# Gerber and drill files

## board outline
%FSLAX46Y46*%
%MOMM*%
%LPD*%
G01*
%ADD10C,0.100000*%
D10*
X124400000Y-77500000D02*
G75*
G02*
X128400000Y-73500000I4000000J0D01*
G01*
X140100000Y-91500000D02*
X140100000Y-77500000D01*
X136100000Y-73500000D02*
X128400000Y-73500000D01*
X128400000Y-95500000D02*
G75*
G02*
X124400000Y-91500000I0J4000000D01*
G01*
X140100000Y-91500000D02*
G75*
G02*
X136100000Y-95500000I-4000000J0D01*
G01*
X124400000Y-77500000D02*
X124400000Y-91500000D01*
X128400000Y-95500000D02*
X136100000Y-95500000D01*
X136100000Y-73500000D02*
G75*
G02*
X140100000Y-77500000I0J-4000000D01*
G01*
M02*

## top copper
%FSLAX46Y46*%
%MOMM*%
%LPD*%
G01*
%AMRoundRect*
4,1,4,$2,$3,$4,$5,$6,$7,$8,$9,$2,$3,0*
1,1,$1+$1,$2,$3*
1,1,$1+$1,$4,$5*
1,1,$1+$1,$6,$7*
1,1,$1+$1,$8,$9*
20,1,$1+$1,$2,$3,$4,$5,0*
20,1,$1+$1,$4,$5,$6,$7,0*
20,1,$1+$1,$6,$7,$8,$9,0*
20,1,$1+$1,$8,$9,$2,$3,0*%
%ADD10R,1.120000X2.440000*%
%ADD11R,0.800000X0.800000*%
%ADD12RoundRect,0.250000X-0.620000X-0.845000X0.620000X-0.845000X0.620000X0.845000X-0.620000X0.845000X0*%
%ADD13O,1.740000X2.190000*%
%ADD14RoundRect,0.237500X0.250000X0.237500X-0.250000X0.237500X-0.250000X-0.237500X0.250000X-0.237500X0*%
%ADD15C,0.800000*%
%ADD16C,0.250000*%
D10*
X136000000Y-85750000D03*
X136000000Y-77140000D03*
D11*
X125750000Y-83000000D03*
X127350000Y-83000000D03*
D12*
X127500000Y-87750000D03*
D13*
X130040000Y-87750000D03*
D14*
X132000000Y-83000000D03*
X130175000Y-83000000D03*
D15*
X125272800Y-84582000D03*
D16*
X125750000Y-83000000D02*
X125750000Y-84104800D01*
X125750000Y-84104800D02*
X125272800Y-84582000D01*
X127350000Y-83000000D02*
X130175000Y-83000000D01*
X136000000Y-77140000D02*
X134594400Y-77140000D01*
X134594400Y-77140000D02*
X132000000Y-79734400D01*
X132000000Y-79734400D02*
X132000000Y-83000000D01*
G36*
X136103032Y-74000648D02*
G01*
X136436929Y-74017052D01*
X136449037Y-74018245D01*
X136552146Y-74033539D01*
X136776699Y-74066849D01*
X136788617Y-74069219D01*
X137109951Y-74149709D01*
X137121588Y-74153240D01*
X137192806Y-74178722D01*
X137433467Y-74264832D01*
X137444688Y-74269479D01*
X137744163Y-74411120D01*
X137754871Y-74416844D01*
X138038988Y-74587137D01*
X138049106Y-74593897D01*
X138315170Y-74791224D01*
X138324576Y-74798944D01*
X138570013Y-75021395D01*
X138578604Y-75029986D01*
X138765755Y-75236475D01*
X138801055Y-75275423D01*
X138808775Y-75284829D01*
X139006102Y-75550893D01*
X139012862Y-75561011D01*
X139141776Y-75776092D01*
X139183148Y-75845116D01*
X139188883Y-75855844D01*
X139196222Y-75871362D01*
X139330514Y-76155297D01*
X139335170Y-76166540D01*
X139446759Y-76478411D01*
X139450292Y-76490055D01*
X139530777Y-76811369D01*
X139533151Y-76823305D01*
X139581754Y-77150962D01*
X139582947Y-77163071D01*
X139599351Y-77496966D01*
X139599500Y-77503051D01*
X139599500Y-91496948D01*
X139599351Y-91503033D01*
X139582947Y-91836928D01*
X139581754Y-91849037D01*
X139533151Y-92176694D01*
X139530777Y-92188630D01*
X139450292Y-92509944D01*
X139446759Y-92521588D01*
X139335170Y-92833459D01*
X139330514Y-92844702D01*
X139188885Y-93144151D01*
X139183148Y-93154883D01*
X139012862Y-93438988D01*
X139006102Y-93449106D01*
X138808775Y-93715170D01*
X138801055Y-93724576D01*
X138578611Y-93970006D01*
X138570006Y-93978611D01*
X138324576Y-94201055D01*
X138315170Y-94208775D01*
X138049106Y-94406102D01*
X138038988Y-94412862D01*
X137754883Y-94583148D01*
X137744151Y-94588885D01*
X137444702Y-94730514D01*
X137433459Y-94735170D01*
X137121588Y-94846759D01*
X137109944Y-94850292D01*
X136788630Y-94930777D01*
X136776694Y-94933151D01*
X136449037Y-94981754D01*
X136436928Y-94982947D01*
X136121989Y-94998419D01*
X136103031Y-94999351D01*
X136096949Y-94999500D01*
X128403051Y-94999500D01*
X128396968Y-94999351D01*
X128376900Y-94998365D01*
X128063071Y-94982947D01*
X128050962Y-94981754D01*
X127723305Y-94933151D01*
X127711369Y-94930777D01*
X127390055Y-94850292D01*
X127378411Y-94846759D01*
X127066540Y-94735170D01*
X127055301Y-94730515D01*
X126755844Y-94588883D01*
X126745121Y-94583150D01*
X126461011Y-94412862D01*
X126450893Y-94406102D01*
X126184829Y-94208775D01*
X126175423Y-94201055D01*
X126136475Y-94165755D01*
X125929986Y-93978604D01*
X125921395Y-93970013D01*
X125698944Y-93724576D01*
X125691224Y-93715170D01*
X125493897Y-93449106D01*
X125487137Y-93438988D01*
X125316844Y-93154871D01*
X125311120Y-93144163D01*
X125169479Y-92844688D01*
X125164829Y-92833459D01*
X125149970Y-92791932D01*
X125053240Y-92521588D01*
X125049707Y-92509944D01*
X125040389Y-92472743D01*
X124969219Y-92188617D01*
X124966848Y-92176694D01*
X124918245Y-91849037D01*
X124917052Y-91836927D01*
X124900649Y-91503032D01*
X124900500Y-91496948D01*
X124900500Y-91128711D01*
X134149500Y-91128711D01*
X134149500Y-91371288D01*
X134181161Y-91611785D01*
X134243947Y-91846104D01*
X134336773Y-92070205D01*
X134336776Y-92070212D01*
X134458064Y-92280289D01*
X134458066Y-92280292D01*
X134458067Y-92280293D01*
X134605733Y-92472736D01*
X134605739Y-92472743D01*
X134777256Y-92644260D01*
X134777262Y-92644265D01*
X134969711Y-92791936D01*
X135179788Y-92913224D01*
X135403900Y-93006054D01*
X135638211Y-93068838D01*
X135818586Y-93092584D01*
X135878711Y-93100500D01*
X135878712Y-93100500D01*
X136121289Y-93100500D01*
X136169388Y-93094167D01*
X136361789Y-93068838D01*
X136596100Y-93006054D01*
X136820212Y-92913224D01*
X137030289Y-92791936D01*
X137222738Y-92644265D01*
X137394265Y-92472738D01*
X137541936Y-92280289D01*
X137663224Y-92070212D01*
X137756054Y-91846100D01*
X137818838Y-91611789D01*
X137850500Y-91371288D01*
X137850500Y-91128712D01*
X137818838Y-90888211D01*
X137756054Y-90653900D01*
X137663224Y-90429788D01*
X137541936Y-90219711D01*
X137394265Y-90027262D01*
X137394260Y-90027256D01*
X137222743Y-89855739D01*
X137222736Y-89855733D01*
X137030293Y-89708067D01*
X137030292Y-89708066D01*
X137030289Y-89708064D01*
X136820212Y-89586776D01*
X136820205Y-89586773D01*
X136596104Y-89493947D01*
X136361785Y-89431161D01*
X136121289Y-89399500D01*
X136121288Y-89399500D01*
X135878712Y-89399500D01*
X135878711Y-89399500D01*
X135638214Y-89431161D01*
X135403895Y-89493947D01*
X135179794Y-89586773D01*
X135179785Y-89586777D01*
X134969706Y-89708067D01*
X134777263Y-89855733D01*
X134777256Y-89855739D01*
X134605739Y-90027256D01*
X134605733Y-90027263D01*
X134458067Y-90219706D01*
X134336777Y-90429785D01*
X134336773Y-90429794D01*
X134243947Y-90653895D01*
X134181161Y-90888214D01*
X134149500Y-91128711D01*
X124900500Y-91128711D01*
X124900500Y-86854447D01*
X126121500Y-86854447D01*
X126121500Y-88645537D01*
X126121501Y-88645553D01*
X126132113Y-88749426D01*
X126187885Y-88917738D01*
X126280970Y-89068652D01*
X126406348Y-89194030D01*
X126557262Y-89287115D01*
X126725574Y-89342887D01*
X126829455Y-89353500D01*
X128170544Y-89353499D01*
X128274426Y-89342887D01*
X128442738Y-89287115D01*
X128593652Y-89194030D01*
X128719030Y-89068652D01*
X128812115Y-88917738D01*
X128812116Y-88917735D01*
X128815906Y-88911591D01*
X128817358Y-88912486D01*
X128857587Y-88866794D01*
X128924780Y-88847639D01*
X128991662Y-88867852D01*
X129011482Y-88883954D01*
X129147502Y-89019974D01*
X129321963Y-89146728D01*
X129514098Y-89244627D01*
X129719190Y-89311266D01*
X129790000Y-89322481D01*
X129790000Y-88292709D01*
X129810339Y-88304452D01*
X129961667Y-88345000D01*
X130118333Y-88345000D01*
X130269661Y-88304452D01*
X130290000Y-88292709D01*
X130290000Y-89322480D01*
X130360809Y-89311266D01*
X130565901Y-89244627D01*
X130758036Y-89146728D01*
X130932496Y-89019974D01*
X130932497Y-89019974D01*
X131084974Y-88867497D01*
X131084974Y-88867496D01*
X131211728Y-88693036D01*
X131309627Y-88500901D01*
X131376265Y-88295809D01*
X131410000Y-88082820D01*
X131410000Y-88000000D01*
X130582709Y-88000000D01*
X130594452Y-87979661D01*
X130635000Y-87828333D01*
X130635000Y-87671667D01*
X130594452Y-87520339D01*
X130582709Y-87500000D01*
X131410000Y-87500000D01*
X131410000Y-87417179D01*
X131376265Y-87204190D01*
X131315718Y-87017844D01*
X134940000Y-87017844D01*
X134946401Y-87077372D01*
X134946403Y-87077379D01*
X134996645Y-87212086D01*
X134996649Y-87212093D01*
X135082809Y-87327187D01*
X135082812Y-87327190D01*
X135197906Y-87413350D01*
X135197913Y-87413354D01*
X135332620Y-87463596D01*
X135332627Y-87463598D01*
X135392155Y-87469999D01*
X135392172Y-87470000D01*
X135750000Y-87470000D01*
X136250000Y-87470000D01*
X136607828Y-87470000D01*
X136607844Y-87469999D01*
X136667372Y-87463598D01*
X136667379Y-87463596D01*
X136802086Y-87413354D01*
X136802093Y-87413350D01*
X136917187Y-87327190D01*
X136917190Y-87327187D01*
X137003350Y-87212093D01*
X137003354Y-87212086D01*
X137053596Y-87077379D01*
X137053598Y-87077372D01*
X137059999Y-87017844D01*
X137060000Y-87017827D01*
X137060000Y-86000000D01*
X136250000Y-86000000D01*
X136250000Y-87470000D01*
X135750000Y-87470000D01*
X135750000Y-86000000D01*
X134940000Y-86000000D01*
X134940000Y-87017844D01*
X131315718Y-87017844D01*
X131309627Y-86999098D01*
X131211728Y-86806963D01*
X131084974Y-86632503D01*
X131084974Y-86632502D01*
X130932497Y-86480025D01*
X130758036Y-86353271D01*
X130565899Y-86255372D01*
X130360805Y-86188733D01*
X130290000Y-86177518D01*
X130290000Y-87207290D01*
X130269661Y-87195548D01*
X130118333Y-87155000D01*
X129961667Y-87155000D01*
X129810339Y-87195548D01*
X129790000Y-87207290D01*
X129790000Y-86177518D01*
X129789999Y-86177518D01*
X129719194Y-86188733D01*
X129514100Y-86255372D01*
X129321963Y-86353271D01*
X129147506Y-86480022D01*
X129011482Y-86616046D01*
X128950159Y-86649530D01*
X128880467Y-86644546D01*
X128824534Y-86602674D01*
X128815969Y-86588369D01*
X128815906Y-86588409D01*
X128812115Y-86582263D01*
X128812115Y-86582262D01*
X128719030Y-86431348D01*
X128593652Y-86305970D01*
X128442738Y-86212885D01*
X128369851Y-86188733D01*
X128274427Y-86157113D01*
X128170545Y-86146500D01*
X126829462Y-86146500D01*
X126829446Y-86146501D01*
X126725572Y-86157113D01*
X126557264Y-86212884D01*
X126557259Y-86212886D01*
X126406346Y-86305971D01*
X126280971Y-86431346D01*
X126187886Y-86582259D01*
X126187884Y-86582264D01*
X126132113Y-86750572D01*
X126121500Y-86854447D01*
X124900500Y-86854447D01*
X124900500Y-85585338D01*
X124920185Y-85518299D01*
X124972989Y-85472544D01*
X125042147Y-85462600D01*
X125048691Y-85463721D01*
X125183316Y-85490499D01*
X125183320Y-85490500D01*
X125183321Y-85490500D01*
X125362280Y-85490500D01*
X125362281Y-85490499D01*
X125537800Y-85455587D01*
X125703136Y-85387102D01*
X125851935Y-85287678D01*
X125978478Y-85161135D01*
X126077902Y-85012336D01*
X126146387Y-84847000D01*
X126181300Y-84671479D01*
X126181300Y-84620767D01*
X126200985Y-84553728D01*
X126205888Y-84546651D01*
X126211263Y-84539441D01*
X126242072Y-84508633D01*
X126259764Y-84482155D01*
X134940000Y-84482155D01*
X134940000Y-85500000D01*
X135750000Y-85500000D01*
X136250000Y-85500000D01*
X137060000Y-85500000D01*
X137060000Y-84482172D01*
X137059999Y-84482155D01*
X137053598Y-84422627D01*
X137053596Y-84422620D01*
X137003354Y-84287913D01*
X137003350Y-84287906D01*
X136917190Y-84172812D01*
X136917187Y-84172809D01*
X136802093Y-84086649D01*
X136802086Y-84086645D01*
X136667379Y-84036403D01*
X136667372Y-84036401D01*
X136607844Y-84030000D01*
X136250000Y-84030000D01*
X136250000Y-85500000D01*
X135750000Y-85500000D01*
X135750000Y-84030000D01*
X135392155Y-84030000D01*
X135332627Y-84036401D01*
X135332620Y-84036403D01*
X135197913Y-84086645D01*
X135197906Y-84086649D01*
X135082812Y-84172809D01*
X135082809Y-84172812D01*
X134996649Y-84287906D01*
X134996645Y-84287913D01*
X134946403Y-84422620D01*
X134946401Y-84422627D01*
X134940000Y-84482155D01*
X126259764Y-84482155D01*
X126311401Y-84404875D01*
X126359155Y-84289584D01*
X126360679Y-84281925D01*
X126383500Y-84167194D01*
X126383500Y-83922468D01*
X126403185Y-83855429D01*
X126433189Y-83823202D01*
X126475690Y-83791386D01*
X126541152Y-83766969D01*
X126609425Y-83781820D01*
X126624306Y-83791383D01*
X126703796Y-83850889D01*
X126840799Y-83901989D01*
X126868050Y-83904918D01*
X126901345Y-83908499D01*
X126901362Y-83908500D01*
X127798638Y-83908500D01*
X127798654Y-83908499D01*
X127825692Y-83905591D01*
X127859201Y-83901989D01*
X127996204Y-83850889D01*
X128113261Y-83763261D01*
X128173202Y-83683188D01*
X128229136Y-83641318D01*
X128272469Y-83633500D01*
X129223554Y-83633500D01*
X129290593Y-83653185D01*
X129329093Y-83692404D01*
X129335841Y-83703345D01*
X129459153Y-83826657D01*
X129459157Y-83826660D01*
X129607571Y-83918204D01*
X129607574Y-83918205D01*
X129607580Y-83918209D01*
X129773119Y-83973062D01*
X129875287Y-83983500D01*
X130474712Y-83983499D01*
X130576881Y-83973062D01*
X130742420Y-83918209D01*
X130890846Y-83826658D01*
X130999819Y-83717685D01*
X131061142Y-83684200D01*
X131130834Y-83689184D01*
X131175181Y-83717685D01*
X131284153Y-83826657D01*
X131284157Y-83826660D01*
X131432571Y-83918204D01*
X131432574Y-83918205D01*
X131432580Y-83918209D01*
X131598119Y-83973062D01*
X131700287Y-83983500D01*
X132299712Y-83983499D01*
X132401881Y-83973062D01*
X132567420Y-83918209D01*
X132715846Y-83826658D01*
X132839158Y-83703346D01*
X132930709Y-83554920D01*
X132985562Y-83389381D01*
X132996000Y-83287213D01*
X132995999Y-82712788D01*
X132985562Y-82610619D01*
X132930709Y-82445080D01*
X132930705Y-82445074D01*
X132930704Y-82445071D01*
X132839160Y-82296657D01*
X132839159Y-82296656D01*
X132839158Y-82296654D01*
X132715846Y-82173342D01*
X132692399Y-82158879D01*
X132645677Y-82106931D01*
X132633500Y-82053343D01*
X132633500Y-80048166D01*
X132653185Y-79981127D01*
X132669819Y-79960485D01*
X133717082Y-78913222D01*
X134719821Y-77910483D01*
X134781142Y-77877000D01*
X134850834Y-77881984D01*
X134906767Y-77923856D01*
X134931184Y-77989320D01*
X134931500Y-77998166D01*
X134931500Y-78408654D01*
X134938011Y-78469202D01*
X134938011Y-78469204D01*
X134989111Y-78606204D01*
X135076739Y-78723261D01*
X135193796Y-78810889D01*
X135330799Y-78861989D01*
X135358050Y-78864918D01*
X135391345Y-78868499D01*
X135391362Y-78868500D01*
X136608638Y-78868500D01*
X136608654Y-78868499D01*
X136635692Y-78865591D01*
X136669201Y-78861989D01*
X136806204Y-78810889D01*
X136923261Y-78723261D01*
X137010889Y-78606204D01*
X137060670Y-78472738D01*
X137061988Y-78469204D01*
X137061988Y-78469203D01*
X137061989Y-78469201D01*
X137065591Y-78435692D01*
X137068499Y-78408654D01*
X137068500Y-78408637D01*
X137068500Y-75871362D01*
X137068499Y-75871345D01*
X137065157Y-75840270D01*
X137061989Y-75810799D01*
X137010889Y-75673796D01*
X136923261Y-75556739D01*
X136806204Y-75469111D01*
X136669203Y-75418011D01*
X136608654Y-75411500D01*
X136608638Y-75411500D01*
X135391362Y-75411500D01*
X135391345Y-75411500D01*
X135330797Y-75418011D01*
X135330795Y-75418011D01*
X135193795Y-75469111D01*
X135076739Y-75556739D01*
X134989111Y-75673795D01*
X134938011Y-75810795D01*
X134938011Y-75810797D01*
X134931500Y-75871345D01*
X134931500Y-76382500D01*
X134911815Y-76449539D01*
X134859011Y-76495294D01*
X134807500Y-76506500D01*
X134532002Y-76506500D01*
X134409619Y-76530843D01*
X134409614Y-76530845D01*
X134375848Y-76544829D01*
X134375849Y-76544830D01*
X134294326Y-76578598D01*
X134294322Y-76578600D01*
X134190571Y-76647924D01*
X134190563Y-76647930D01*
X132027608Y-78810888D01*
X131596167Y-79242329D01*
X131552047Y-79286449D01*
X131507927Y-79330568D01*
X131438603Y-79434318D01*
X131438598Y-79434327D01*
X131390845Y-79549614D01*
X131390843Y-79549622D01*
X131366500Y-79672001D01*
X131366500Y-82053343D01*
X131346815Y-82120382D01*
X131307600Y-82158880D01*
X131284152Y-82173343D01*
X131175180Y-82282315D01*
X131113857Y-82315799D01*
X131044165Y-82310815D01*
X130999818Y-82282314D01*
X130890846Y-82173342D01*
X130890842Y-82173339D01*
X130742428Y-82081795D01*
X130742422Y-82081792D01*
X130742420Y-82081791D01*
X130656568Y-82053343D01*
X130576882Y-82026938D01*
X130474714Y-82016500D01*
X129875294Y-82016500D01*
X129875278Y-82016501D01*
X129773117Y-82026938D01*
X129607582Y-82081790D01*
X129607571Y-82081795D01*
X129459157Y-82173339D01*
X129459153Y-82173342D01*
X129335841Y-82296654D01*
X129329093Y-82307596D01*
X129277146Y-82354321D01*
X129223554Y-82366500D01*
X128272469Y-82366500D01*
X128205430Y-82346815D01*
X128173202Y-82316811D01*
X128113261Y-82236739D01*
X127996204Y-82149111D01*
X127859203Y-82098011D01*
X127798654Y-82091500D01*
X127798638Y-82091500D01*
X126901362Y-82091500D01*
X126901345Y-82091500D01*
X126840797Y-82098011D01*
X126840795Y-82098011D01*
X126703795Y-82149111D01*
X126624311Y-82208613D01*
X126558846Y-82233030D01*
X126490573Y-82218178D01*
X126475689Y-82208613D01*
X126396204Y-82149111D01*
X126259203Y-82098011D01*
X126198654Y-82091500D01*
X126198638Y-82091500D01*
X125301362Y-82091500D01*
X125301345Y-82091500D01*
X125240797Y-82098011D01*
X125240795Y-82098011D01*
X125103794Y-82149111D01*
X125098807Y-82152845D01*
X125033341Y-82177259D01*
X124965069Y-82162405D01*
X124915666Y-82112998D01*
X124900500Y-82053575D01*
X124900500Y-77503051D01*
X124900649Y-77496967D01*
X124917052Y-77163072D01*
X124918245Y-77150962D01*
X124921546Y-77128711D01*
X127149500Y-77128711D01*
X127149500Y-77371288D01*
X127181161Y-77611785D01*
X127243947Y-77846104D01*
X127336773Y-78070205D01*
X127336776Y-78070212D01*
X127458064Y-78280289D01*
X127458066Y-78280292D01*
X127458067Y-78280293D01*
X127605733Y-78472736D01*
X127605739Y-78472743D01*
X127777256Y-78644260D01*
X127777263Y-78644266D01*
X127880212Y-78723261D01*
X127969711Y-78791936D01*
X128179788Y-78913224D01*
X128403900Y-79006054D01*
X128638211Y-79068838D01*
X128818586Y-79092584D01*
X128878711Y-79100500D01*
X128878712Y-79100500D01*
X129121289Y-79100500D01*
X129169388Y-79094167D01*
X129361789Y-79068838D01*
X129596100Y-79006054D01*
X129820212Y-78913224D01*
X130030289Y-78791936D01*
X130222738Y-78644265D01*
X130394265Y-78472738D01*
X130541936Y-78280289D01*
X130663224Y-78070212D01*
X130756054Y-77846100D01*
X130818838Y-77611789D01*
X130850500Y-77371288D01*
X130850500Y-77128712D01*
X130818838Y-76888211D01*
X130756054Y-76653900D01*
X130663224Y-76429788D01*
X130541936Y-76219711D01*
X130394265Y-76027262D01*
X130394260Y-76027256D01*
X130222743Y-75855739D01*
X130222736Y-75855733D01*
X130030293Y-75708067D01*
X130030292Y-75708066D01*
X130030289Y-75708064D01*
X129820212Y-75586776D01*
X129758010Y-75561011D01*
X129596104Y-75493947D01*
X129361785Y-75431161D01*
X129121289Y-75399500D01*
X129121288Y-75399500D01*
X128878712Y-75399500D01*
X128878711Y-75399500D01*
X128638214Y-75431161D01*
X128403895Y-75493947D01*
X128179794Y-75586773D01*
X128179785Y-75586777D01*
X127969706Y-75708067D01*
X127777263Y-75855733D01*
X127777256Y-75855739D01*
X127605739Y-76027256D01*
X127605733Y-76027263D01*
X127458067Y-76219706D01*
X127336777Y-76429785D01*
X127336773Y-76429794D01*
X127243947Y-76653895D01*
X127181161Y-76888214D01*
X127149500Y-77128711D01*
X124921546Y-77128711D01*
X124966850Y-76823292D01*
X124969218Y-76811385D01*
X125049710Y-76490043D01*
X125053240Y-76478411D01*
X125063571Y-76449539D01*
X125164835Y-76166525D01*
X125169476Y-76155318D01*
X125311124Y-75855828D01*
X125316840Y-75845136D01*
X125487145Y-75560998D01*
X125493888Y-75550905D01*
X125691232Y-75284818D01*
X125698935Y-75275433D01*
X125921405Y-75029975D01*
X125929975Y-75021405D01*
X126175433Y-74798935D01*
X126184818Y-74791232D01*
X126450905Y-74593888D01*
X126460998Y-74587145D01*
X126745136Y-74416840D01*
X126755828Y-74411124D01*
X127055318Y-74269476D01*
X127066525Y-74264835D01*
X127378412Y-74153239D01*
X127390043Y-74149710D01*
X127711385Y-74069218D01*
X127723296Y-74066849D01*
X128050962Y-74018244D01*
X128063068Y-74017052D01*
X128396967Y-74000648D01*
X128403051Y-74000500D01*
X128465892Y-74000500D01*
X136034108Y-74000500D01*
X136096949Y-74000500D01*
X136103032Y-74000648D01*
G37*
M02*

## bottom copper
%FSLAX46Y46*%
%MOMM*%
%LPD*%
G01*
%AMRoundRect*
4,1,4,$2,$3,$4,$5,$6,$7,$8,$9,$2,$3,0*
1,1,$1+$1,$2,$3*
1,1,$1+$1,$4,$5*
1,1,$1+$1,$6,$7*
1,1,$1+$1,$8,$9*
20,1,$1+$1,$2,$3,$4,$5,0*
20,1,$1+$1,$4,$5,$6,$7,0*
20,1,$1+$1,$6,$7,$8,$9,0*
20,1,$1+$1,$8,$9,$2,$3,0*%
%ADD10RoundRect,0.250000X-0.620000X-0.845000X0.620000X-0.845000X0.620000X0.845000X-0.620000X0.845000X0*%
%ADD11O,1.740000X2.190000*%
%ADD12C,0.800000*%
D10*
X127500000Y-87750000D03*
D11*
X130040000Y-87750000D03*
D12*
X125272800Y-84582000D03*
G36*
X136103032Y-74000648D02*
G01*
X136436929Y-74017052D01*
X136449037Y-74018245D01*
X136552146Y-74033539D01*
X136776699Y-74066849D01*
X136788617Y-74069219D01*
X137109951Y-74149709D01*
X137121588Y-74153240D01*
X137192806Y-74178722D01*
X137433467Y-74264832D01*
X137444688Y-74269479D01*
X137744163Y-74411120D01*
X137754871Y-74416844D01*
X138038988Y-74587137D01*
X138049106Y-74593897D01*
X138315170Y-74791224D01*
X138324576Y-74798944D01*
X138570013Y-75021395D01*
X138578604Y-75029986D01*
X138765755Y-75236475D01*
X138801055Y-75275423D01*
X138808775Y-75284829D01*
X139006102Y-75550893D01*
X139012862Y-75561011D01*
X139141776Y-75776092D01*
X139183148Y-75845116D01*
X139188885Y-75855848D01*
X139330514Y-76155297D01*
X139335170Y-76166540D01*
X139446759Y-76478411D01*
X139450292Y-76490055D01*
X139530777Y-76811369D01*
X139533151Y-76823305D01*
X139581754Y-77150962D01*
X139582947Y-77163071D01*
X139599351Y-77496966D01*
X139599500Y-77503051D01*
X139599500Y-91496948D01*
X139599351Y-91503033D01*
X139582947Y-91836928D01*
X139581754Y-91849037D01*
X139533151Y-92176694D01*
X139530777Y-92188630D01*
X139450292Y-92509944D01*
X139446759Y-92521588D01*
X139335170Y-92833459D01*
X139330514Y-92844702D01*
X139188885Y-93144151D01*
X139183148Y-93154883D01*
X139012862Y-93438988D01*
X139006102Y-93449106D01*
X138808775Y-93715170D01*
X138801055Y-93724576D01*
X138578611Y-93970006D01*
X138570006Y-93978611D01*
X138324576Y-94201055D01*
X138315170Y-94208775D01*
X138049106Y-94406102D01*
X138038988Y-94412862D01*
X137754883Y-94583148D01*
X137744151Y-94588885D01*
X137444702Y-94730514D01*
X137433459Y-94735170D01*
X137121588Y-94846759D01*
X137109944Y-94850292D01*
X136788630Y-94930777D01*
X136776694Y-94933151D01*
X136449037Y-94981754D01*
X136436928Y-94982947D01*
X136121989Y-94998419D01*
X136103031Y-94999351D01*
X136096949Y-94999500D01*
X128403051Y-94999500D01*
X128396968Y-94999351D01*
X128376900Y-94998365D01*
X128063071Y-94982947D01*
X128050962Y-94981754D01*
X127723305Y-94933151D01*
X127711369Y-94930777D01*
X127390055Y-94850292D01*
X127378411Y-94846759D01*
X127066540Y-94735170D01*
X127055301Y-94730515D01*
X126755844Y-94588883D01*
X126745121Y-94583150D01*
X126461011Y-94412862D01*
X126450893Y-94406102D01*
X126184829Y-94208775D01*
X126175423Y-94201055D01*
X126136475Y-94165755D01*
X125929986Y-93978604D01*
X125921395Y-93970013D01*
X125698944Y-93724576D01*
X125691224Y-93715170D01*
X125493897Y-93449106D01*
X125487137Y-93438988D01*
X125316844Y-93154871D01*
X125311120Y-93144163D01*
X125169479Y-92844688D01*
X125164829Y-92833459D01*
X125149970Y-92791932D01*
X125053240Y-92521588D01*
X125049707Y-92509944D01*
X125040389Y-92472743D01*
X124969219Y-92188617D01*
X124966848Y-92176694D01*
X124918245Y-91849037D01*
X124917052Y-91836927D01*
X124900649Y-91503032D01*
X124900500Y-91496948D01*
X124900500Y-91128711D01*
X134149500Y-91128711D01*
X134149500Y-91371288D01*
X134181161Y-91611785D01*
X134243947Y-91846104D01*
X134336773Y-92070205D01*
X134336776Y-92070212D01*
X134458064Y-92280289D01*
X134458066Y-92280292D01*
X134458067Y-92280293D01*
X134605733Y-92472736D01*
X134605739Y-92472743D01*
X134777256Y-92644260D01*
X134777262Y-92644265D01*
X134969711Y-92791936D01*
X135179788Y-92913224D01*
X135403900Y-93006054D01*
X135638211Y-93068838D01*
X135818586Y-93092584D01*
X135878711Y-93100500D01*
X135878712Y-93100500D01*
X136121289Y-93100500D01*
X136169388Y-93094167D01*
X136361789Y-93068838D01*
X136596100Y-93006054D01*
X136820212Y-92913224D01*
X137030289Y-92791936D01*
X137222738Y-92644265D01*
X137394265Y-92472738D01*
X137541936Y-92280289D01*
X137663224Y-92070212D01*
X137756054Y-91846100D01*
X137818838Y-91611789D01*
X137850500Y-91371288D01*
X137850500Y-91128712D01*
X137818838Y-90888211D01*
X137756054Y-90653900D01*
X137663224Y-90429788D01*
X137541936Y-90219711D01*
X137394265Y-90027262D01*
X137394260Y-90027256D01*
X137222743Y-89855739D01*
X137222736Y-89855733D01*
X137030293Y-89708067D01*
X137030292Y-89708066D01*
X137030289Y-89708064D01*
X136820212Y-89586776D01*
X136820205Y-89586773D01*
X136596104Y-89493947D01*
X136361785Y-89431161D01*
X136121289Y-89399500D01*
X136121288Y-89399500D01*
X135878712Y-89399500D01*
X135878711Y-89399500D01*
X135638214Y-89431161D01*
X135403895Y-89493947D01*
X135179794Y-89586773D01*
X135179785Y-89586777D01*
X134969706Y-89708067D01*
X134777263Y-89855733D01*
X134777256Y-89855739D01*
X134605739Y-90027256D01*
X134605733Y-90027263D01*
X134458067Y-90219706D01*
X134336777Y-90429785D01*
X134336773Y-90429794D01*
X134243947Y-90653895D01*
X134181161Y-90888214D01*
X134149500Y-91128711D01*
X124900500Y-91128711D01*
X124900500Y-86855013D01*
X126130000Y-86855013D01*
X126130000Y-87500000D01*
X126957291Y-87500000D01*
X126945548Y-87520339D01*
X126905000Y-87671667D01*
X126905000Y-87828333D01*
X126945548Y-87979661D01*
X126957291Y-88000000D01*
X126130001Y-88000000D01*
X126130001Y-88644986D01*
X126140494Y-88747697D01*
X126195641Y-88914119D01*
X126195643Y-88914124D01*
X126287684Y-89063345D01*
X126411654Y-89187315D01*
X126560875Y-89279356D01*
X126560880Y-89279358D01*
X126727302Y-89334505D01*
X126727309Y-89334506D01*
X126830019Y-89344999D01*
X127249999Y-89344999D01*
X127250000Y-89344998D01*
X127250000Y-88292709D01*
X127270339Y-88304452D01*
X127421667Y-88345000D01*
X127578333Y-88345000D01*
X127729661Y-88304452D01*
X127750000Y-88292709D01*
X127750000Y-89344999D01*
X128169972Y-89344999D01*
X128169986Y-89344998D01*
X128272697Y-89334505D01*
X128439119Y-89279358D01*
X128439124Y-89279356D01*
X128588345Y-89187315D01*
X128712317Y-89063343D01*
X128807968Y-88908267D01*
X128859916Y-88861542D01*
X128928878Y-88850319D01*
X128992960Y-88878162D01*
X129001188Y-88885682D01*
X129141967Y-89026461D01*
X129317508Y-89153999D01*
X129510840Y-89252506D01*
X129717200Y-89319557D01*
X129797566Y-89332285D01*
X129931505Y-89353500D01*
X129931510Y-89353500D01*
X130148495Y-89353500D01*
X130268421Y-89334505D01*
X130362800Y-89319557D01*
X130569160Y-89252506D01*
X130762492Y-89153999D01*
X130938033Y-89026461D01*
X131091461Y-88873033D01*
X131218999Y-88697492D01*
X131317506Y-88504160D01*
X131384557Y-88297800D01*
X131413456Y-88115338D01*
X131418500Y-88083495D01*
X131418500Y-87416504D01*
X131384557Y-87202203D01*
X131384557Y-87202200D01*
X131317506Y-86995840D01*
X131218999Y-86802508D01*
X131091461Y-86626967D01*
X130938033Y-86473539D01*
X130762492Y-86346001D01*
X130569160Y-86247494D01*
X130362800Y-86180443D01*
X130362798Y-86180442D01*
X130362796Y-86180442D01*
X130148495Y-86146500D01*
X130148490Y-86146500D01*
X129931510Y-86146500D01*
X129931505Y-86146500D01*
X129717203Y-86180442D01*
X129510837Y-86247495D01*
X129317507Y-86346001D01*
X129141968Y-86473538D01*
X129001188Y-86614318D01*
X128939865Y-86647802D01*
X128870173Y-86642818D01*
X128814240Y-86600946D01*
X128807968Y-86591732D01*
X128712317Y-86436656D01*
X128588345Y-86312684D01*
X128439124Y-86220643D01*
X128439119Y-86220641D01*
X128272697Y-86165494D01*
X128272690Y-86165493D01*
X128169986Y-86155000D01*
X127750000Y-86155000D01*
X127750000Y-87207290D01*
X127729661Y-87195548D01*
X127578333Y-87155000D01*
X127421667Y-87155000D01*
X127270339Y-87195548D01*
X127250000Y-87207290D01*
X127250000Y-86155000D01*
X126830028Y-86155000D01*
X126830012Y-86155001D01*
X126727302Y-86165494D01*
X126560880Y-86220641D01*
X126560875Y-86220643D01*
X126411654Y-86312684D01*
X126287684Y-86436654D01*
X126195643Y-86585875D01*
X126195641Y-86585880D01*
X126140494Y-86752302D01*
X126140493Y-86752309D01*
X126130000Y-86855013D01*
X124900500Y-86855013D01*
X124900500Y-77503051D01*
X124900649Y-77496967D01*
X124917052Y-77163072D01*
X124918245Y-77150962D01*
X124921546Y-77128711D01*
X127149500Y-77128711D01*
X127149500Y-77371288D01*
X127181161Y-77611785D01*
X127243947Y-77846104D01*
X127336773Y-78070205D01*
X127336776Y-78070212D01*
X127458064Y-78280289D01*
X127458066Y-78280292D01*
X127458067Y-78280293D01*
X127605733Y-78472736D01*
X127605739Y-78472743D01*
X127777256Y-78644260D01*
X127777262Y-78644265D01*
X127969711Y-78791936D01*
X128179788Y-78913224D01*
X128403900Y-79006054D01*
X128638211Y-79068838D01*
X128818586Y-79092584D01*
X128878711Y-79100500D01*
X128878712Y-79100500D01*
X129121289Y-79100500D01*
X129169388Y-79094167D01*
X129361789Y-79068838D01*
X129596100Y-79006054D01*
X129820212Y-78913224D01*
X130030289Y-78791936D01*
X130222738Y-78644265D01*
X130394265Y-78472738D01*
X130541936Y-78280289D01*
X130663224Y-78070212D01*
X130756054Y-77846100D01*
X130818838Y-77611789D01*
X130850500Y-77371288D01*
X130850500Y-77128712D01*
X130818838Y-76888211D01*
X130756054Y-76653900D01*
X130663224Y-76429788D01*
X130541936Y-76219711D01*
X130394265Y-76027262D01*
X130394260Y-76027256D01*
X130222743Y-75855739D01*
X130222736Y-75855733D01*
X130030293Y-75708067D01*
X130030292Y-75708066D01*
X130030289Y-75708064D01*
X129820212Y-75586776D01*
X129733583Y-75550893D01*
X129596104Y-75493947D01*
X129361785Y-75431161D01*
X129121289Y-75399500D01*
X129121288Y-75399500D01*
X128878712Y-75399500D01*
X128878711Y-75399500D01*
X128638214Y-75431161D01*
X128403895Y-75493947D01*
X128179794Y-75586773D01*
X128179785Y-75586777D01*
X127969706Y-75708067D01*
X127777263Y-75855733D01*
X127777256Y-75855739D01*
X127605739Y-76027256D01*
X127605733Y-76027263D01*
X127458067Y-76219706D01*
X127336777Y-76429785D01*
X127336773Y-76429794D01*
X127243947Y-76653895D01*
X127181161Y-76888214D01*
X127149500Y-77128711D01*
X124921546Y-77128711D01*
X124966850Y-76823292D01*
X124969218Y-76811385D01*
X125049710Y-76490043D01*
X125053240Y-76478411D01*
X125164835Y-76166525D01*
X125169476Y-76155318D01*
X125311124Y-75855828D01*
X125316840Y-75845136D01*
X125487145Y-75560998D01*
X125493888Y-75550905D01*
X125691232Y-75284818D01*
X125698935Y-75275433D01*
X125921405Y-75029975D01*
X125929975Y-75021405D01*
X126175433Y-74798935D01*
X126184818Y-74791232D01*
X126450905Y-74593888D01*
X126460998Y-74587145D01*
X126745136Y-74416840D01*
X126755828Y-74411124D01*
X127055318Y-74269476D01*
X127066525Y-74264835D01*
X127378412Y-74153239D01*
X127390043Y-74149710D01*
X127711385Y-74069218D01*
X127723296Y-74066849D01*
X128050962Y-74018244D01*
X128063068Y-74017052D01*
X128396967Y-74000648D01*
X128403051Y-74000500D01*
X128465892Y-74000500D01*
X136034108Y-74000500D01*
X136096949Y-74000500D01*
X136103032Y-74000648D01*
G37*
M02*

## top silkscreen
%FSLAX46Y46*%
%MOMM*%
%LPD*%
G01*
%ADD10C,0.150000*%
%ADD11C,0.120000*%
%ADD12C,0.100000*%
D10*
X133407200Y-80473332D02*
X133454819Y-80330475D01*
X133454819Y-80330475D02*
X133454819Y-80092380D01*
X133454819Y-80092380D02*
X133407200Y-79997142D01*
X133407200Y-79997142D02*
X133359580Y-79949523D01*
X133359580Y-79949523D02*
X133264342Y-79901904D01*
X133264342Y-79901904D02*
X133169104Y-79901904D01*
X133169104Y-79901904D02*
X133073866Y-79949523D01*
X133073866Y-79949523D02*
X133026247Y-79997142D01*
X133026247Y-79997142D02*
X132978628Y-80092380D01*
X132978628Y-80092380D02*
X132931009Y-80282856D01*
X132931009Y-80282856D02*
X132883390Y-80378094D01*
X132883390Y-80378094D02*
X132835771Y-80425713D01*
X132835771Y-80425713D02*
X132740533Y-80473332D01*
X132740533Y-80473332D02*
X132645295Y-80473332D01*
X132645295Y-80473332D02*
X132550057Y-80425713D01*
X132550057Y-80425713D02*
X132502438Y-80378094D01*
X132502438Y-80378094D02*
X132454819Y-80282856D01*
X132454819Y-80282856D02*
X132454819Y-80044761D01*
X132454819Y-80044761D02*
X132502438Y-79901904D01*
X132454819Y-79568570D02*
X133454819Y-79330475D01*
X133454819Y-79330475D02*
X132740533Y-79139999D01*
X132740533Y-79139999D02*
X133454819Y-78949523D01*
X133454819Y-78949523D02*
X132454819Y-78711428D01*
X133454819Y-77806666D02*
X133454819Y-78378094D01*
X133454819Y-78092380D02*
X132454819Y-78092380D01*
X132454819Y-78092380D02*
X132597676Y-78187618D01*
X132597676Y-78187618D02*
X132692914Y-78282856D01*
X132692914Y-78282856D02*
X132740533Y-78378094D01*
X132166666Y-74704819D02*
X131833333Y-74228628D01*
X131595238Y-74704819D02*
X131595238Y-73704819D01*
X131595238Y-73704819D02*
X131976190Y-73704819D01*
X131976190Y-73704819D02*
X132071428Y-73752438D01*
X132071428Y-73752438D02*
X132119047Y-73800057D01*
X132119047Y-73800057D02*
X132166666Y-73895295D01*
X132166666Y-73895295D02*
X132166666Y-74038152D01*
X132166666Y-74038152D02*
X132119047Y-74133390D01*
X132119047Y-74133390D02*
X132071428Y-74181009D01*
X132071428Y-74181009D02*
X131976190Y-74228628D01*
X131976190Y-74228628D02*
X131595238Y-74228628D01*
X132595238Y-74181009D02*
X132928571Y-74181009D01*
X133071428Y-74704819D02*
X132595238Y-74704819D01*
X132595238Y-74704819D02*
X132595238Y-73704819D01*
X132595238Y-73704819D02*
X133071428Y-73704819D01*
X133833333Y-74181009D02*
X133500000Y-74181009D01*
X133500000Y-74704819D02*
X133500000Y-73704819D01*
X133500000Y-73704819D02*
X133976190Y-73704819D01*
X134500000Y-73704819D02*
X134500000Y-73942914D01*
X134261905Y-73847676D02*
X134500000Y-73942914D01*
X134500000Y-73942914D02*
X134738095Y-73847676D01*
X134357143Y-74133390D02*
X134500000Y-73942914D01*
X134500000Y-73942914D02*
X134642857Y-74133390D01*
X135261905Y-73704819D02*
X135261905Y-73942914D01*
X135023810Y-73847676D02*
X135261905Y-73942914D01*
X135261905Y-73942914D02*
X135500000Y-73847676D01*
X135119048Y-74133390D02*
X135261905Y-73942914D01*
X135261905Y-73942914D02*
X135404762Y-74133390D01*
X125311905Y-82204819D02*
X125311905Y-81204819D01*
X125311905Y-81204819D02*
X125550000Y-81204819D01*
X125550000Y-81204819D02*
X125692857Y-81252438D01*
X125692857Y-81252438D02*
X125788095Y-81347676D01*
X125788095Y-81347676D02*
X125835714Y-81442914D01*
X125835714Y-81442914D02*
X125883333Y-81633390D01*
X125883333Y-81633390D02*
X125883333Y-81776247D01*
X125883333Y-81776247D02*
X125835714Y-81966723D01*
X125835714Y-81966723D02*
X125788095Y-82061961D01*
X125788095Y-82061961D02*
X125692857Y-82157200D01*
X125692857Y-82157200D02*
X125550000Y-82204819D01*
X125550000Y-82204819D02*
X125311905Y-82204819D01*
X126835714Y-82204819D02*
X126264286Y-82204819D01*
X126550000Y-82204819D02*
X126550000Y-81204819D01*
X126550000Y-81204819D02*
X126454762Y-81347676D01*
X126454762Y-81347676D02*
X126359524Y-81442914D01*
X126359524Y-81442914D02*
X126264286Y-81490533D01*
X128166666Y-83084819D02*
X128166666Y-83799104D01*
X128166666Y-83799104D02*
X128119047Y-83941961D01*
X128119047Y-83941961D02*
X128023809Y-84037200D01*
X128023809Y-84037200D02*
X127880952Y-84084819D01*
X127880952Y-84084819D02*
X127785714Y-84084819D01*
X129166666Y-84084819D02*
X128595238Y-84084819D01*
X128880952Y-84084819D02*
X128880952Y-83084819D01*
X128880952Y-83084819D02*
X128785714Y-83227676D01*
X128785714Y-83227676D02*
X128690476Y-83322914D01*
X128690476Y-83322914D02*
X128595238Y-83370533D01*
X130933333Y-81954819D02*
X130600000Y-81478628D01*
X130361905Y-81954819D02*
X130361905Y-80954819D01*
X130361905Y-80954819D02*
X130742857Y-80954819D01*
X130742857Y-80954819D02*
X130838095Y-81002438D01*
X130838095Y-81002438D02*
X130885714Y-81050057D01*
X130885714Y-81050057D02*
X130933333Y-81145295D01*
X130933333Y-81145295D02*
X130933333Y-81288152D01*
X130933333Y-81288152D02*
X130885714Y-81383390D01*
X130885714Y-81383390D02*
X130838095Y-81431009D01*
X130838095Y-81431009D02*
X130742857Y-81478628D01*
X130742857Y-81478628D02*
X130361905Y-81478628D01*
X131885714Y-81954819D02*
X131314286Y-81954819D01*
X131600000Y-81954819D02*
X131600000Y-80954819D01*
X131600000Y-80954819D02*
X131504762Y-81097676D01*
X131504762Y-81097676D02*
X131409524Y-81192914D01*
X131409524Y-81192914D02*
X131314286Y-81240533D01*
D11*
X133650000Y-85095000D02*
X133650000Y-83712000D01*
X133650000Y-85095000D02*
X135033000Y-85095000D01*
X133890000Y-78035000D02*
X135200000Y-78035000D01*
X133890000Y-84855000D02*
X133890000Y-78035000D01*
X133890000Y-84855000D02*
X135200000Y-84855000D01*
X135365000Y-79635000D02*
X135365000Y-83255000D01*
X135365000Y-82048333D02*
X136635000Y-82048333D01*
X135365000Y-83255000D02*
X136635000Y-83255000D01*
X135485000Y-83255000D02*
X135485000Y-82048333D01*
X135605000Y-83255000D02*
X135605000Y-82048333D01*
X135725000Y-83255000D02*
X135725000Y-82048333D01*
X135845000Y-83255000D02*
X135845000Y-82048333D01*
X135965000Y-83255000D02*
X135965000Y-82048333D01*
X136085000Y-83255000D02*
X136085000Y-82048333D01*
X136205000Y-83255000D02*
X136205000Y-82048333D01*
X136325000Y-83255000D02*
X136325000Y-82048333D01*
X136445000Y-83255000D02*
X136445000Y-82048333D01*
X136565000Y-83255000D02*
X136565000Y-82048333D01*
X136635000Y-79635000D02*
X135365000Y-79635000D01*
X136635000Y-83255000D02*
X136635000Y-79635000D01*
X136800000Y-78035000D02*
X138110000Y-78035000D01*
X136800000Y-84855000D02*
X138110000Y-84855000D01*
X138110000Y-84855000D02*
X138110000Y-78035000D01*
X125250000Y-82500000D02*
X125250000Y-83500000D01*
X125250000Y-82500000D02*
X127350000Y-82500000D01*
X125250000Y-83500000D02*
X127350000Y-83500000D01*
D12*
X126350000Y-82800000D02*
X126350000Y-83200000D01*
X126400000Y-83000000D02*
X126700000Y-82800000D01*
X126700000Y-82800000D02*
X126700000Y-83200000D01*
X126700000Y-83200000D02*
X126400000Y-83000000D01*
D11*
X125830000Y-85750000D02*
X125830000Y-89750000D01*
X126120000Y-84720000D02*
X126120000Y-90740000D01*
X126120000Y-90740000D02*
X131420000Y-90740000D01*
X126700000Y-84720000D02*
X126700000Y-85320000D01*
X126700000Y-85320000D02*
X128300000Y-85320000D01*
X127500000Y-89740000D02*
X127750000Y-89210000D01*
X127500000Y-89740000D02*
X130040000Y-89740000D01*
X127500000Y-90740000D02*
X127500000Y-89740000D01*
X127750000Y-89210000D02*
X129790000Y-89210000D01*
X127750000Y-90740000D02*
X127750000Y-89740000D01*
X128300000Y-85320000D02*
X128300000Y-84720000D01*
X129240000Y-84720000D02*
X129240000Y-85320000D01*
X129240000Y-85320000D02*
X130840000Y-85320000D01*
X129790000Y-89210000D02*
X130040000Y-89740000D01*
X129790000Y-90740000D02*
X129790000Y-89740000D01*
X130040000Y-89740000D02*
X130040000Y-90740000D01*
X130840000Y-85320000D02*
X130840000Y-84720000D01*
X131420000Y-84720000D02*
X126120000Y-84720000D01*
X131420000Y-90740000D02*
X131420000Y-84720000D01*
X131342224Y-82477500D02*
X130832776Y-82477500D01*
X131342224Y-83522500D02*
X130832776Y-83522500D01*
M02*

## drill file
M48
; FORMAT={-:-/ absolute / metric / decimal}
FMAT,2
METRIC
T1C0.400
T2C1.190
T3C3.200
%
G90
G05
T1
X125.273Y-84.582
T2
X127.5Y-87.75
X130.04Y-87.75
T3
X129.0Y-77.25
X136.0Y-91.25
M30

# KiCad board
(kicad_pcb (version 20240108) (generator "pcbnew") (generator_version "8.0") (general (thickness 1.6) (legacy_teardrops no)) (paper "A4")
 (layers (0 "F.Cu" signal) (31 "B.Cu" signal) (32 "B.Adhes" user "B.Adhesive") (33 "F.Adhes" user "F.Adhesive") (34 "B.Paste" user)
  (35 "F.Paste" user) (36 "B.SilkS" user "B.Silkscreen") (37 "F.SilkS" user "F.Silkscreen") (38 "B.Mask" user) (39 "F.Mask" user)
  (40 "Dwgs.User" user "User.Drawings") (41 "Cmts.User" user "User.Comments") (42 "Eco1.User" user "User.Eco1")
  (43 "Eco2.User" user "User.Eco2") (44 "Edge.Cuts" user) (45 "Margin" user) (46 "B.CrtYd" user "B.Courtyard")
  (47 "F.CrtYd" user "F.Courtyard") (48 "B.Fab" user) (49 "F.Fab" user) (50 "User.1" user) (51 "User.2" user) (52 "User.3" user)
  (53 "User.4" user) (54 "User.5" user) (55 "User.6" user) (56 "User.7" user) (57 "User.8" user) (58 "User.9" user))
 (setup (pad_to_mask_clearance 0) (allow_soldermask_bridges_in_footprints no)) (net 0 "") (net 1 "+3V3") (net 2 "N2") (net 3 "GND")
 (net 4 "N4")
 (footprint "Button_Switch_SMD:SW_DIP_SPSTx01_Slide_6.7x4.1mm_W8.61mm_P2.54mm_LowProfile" (layer "F.Cu") (at 136 81.445 90)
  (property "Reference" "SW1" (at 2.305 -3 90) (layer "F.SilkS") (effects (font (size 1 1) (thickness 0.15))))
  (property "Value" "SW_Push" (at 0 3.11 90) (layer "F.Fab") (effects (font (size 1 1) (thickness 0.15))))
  (fp_line (start -3.65 -2.35) (end -2.267 -2.35) (stroke (width 0.12) (type solid)) (layer "F.SilkS"))
  (fp_line (start -3.65 -2.35) (end -3.65 -0.967) (stroke (width 0.12) (type solid)) (layer "F.SilkS"))
  (fp_line (start 3.41 -2.11) (end 3.41 -0.8) (stroke (width 0.12) (type solid)) (layer "F.SilkS"))
  (fp_line (start -3.41 -2.11) (end 3.41 -2.11) (stroke (width 0.12) (type solid)) (layer "F.SilkS"))
  (fp_line (start -3.41 -2.11) (end -3.41 -0.8) (stroke (width 0.12) (type solid)) (layer "F.SilkS"))
  (fp_line (start 1.81 -0.635) (end -1.81 -0.635) (stroke (width 0.12) (type solid)) (layer "F.SilkS"))
  (fp_line (start -0.603333 -0.635) (end -0.603333 0.635) (stroke (width 0.12) (type solid)) (layer "F.SilkS"))
  (fp_line (start -1.81 -0.635) (end -1.81 0.635) (stroke (width 0.12) (type solid)) (layer "F.SilkS"))
  (fp_line (start -1.81 -0.515) (end -0.603333 -0.515) (stroke (width 0.12) (type solid)) (layer "F.SilkS"))
  (fp_line (start -1.81 -0.395) (end -0.603333 -0.395) (stroke (width 0.12) (type solid)) (layer "F.SilkS"))
  (fp_line (start -1.81 -0.275) (end -0.603333 -0.275) (stroke (width 0.12) (type solid)) (layer "F.SilkS"))
  (fp_line (start -1.81 -0.155) (end -0.603333 -0.155) (stroke (width 0.12) (type solid)) (layer "F.SilkS"))
  (fp_line (start -1.81 -0.035) (end -0.603333 -0.035) (stroke (width 0.12) (type solid)) (layer "F.SilkS"))
  (fp_line (start -1.81 0.085) (end -0.603333 0.085) (stroke (width 0.12) (type solid)) (layer "F.SilkS"))
  (fp_line (start -1.81 0.205) (end -0.603333 0.205) (stroke (width 0.12) (type solid)) (layer "F.SilkS"))
  (fp_line (start -1.81 0.325) (end -0.603333 0.325) (stroke (width 0.12) (type solid)) (layer "F.SilkS"))
  (fp_line (start -1.81 0.445) (end -0.603333 0.445) (stroke (width 0.12) (type solid)) (layer "F.SilkS"))
  (fp_line (start -1.81 0.565) (end -0.603333 0.565) (stroke (width 0.12) (type solid)) (layer "F.SilkS"))
  (fp_line (start 1.81 0.635) (end 1.81 -0.635) (stroke (width 0.12) (type solid)) (layer "F.SilkS"))
  (fp_line (start -1.81 0.635) (end 1.81 0.635) (stroke (width 0.12) (type solid)) (layer "F.SilkS"))
  (fp_line (start 3.41 0.8) (end 3.41 2.11) (stroke (width 0.12) (type solid)) (layer "F.SilkS"))
  (fp_line (start -3.41 0.8) (end -3.41 2.11) (stroke (width 0.12) (type solid)) (layer "F.SilkS"))
  (fp_line (start -3.41 2.11) (end 3.41 2.11) (stroke (width 0.12) (type solid)) (layer "F.SilkS"))
  (pad "1" smd rect (at -4.305 0 90) (size 2.44 1.12) (layers "F.Cu" "F.Paste" "F.Mask") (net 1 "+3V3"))
  (pad "2" smd rect (at 4.305 0 90) (size 2.44 1.12) (layers "F.Cu" "F.Paste" "F.Mask") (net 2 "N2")))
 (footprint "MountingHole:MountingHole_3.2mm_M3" (layer "F.Cu") (at 129 77.25)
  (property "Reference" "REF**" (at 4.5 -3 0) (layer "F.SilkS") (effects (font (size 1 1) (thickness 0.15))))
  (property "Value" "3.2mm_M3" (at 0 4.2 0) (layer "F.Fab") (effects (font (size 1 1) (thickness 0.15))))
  (pad "" np_thru_hole circle (at 0 0) (size 3.2 3.2) (drill 3.2) (layers "*.Cu" "*.Mask")))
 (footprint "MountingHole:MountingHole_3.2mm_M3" (layer "F.Cu") (at 136 91.25)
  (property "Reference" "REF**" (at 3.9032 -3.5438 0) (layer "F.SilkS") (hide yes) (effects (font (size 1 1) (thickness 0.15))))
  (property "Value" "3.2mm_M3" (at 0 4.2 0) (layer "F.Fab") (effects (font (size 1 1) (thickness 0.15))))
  (pad "" np_thru_hole circle (at 0 0) (size 3.2 3.2) (drill 3.2) (layers "*.Cu" "*.Mask")))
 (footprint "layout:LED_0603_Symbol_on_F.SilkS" (layer "F.Cu") (at 126.55 83)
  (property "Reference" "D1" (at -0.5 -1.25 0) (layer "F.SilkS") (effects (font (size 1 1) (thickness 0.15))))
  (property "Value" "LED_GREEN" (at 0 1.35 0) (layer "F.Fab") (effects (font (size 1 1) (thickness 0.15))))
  (fp_line (start -1.3 -0.5) (end -1.3 0.5) (stroke (width 0.12) (type solid)) (layer "F.SilkS"))
  (fp_line (start -1.3 -0.5) (end 0.8 -0.5) (stroke (width 0.12) (type solid)) (layer "F.SilkS"))
  (fp_line (start -1.3 0.5) (end 0.8 0.5) (stroke (width 0.12) (type solid)) (layer "F.SilkS"))
  (fp_line (start -0.2 -0.2) (end -0.2 0.2) (stroke (width 0.1) (type solid)) (layer "F.SilkS"))
  (fp_line (start -0.15 0) (end 0.15 -0.2) (stroke (width 0.1) (type solid)) (layer "F.SilkS"))
  (fp_line (start 0.15 -0.2) (end 0.15 0.2) (stroke (width 0.1) (type solid)) (layer "F.SilkS"))
  (fp_line (start 0.15 0.2) (end -0.15 0) (stroke (width 0.1) (type solid)) (layer "F.SilkS"))
  (pad "1" smd rect (at -0.8 0 180) (size 0.8 0.8) (layers "F.Cu" "F.Paste" "F.Mask") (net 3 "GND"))
  (pad "2" smd rect (at 0.8 0 180) (size 0.8 0.8) (layers "F.Cu" "F.Paste" "F.Mask") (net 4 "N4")))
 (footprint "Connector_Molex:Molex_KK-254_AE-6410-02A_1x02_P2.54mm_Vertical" (layer "F.Cu") (at 127.5 87.75)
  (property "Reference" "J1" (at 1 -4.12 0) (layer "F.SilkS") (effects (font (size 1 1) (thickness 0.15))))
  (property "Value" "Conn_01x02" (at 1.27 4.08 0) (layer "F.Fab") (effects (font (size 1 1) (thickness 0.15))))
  (fp_line (start -1.67 -2) (end -1.67 2) (stroke (width 0.12) (type solid)) (layer "F.SilkS"))
  (fp_line (start -1.38 -3.03) (end -1.38 2.99) (stroke (width 0.12) (type solid)) (layer "F.SilkS"))
  (fp_line (start -1.38 2.99) (end 3.92 2.99) (stroke (width 0.12) (type solid)) (layer "F.SilkS"))
  (fp_line (start -0.8 -3.03) (end -0.8 -2.43) (stroke (width 0.12) (type solid)) (layer "F.SilkS"))
  (fp_line (start -0.8 -2.43) (end 0.8 -2.43) (stroke (width 0.12) (type solid)) (layer "F.SilkS"))
  (fp_line (start 0 1.99) (end 0.25 1.46) (stroke (width 0.12) (type solid)) (layer "F.SilkS"))
  (fp_line (start 0 1.99) (end 2.54 1.99) (stroke (width 0.12) (type solid)) (layer "F.SilkS"))
  (fp_line (start 0 2.99) (end 0 1.99) (stroke (width 0.12) (type solid)) (layer "F.SilkS"))
  (fp_line (start 0.25 1.46) (end 2.29 1.46) (stroke (width 0.12) (type solid)) (layer "F.SilkS"))
  (fp_line (start 0.25 2.99) (end 0.25 1.99) (stroke (width 0.12) (type solid)) (layer "F.SilkS"))
  (fp_line (start 0.8 -2.43) (end 0.8 -3.03) (stroke (width 0.12) (type solid)) (layer "F.SilkS"))
  (fp_line (start 1.74 -3.03) (end 1.74 -2.43) (stroke (width 0.12) (type solid)) (layer "F.SilkS"))
  (fp_line (start 1.74 -2.43) (end 3.34 -2.43) (stroke (width 0.12) (type solid)) (layer "F.SilkS"))
  (fp_line (start 2.29 1.46) (end 2.54 1.99) (stroke (width 0.12) (type solid)) (layer "F.SilkS"))
  (fp_line (start 2.29 2.99) (end 2.29 1.99) (stroke (width 0.12) (type solid)) (layer "F.SilkS"))
  (fp_line (start 2.54 1.99) (end 2.54 2.99) (stroke (width 0.12) (type solid)) (layer "F.SilkS"))
  (fp_line (start 3.34 -2.43) (end 3.34 -3.03) (stroke (width 0.12) (type solid)) (layer "F.SilkS"))
  (fp_line (start 3.92 -3.03) (end -1.38 -3.03) (stroke (width 0.12) (type solid)) (layer "F.SilkS"))
  (fp_line (start 3.92 2.99) (end 3.92 -3.03) (stroke (width 0.12) (type solid)) (layer "F.SilkS"))
  (pad "1" thru_hole roundrect (at 0 0) (size 1.74 2.19) (drill 1.19) (layers "*.Cu" "*.Mask") (remove_unused_layers no)
   (roundrect_rratio 0.143678) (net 3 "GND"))
  (pad "2" thru_hole oval (at 2.54 0) (size 1.74 2.19) (drill 1.19) (layers "*.Cu" "*.Mask") (remove_unused_layers no) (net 1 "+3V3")))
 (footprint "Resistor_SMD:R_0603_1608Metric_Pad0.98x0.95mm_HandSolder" (layer "F.Cu") (at 131.0875 83 180)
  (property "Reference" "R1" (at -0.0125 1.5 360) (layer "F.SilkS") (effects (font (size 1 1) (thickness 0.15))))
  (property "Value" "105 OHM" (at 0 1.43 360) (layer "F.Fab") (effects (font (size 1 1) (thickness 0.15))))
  (fp_line (start -0.254724 0.5225) (end 0.254724 0.5225) (stroke (width 0.12) (type solid)) (layer "F.SilkS"))
  (fp_line (start -0.254724 -0.5225) (end 0.254724 -0.5225) (stroke (width 0.12) (type solid)) (layer "F.SilkS"))
  (pad "1" smd roundrect (at -0.9125 0 180) (size 0.975 0.95) (layers "F.Cu" "F.Paste" "F.Mask") (roundrect_rratio 0.25) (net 2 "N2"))
  (pad "2" smd roundrect (at 0.9125 0 180) (size 0.975 0.95) (layers "F.Cu" "F.Paste" "F.Mask") (roundrect_rratio 0.25) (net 4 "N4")))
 (gr_arc (start 124.4 77.5) (mid 125.571573 74.671573) (end 128.4 73.5) (stroke (width 0.1) (type default)) (layer "Edge.Cuts"))
 (gr_line (start 140.1 91.5) (end 140.1 77.5) (stroke (width 0.1) (type default)) (layer "Edge.Cuts"))
 (gr_line (start 136.1 73.5) (end 128.4 73.5) (stroke (width 0.1) (type default)) (layer "Edge.Cuts"))
 (gr_arc (start 128.4 95.5) (mid 125.571573 94.328427) (end 124.4 91.5) (stroke (width 0.1) (type default)) (layer "Edge.Cuts"))
 (gr_arc (start 140.1 91.5) (mid 138.928427 94.328427) (end 136.1 95.5) (stroke (width 0.1) (type default)) (layer "Edge.Cuts"))
 (gr_line (start 124.4 77.5) (end 124.4 91.5) (stroke (width 0.1) (type default)) (layer "Edge.Cuts"))
 (gr_line (start 128.4 95.5) (end 136.1 95.5) (stroke (width 0.1) (type default)) (layer "Edge.Cuts"))
 (gr_arc (start 136.1 73.5) (mid 138.928427 74.671573) (end 140.1 77.5) (stroke (width 0.1) (type default)) (layer "Edge.Cuts"))
 (segment (start 125.75 83) (end 125.75 84.1048) (width 0.25) (layer "F.Cu") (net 3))
 (segment (start 125.75 84.1048) (end 125.2728 84.582) (width 0.25) (layer "F.Cu") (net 3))
 (via (at 125.2728 84.582) (size 0.8) (drill 0.4) (layers "F.Cu" "B.Cu") (free yes) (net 3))
 (segment (start 127.35 83) (end 130.175 83) (width 0.25) (layer "F.Cu") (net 4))
 (segment (start 136 77.14) (end 134.5944 77.14) (width 0.25) (layer "F.Cu") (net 2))
 (segment (start 134.5944 77.14) (end 132 79.7344) (width 0.25) (layer "F.Cu") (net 2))
 (segment (start 132 79.7344) (end 132 83) (width 0.25) (layer "F.Cu") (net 2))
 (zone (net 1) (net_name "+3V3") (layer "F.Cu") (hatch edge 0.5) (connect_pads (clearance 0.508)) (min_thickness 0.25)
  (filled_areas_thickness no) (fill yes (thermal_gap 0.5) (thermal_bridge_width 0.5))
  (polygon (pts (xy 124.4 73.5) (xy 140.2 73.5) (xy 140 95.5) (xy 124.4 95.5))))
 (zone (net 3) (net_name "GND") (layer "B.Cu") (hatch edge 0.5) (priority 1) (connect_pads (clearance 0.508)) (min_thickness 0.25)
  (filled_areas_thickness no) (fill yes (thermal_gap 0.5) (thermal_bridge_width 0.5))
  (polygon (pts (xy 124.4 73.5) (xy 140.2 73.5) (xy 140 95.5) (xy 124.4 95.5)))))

